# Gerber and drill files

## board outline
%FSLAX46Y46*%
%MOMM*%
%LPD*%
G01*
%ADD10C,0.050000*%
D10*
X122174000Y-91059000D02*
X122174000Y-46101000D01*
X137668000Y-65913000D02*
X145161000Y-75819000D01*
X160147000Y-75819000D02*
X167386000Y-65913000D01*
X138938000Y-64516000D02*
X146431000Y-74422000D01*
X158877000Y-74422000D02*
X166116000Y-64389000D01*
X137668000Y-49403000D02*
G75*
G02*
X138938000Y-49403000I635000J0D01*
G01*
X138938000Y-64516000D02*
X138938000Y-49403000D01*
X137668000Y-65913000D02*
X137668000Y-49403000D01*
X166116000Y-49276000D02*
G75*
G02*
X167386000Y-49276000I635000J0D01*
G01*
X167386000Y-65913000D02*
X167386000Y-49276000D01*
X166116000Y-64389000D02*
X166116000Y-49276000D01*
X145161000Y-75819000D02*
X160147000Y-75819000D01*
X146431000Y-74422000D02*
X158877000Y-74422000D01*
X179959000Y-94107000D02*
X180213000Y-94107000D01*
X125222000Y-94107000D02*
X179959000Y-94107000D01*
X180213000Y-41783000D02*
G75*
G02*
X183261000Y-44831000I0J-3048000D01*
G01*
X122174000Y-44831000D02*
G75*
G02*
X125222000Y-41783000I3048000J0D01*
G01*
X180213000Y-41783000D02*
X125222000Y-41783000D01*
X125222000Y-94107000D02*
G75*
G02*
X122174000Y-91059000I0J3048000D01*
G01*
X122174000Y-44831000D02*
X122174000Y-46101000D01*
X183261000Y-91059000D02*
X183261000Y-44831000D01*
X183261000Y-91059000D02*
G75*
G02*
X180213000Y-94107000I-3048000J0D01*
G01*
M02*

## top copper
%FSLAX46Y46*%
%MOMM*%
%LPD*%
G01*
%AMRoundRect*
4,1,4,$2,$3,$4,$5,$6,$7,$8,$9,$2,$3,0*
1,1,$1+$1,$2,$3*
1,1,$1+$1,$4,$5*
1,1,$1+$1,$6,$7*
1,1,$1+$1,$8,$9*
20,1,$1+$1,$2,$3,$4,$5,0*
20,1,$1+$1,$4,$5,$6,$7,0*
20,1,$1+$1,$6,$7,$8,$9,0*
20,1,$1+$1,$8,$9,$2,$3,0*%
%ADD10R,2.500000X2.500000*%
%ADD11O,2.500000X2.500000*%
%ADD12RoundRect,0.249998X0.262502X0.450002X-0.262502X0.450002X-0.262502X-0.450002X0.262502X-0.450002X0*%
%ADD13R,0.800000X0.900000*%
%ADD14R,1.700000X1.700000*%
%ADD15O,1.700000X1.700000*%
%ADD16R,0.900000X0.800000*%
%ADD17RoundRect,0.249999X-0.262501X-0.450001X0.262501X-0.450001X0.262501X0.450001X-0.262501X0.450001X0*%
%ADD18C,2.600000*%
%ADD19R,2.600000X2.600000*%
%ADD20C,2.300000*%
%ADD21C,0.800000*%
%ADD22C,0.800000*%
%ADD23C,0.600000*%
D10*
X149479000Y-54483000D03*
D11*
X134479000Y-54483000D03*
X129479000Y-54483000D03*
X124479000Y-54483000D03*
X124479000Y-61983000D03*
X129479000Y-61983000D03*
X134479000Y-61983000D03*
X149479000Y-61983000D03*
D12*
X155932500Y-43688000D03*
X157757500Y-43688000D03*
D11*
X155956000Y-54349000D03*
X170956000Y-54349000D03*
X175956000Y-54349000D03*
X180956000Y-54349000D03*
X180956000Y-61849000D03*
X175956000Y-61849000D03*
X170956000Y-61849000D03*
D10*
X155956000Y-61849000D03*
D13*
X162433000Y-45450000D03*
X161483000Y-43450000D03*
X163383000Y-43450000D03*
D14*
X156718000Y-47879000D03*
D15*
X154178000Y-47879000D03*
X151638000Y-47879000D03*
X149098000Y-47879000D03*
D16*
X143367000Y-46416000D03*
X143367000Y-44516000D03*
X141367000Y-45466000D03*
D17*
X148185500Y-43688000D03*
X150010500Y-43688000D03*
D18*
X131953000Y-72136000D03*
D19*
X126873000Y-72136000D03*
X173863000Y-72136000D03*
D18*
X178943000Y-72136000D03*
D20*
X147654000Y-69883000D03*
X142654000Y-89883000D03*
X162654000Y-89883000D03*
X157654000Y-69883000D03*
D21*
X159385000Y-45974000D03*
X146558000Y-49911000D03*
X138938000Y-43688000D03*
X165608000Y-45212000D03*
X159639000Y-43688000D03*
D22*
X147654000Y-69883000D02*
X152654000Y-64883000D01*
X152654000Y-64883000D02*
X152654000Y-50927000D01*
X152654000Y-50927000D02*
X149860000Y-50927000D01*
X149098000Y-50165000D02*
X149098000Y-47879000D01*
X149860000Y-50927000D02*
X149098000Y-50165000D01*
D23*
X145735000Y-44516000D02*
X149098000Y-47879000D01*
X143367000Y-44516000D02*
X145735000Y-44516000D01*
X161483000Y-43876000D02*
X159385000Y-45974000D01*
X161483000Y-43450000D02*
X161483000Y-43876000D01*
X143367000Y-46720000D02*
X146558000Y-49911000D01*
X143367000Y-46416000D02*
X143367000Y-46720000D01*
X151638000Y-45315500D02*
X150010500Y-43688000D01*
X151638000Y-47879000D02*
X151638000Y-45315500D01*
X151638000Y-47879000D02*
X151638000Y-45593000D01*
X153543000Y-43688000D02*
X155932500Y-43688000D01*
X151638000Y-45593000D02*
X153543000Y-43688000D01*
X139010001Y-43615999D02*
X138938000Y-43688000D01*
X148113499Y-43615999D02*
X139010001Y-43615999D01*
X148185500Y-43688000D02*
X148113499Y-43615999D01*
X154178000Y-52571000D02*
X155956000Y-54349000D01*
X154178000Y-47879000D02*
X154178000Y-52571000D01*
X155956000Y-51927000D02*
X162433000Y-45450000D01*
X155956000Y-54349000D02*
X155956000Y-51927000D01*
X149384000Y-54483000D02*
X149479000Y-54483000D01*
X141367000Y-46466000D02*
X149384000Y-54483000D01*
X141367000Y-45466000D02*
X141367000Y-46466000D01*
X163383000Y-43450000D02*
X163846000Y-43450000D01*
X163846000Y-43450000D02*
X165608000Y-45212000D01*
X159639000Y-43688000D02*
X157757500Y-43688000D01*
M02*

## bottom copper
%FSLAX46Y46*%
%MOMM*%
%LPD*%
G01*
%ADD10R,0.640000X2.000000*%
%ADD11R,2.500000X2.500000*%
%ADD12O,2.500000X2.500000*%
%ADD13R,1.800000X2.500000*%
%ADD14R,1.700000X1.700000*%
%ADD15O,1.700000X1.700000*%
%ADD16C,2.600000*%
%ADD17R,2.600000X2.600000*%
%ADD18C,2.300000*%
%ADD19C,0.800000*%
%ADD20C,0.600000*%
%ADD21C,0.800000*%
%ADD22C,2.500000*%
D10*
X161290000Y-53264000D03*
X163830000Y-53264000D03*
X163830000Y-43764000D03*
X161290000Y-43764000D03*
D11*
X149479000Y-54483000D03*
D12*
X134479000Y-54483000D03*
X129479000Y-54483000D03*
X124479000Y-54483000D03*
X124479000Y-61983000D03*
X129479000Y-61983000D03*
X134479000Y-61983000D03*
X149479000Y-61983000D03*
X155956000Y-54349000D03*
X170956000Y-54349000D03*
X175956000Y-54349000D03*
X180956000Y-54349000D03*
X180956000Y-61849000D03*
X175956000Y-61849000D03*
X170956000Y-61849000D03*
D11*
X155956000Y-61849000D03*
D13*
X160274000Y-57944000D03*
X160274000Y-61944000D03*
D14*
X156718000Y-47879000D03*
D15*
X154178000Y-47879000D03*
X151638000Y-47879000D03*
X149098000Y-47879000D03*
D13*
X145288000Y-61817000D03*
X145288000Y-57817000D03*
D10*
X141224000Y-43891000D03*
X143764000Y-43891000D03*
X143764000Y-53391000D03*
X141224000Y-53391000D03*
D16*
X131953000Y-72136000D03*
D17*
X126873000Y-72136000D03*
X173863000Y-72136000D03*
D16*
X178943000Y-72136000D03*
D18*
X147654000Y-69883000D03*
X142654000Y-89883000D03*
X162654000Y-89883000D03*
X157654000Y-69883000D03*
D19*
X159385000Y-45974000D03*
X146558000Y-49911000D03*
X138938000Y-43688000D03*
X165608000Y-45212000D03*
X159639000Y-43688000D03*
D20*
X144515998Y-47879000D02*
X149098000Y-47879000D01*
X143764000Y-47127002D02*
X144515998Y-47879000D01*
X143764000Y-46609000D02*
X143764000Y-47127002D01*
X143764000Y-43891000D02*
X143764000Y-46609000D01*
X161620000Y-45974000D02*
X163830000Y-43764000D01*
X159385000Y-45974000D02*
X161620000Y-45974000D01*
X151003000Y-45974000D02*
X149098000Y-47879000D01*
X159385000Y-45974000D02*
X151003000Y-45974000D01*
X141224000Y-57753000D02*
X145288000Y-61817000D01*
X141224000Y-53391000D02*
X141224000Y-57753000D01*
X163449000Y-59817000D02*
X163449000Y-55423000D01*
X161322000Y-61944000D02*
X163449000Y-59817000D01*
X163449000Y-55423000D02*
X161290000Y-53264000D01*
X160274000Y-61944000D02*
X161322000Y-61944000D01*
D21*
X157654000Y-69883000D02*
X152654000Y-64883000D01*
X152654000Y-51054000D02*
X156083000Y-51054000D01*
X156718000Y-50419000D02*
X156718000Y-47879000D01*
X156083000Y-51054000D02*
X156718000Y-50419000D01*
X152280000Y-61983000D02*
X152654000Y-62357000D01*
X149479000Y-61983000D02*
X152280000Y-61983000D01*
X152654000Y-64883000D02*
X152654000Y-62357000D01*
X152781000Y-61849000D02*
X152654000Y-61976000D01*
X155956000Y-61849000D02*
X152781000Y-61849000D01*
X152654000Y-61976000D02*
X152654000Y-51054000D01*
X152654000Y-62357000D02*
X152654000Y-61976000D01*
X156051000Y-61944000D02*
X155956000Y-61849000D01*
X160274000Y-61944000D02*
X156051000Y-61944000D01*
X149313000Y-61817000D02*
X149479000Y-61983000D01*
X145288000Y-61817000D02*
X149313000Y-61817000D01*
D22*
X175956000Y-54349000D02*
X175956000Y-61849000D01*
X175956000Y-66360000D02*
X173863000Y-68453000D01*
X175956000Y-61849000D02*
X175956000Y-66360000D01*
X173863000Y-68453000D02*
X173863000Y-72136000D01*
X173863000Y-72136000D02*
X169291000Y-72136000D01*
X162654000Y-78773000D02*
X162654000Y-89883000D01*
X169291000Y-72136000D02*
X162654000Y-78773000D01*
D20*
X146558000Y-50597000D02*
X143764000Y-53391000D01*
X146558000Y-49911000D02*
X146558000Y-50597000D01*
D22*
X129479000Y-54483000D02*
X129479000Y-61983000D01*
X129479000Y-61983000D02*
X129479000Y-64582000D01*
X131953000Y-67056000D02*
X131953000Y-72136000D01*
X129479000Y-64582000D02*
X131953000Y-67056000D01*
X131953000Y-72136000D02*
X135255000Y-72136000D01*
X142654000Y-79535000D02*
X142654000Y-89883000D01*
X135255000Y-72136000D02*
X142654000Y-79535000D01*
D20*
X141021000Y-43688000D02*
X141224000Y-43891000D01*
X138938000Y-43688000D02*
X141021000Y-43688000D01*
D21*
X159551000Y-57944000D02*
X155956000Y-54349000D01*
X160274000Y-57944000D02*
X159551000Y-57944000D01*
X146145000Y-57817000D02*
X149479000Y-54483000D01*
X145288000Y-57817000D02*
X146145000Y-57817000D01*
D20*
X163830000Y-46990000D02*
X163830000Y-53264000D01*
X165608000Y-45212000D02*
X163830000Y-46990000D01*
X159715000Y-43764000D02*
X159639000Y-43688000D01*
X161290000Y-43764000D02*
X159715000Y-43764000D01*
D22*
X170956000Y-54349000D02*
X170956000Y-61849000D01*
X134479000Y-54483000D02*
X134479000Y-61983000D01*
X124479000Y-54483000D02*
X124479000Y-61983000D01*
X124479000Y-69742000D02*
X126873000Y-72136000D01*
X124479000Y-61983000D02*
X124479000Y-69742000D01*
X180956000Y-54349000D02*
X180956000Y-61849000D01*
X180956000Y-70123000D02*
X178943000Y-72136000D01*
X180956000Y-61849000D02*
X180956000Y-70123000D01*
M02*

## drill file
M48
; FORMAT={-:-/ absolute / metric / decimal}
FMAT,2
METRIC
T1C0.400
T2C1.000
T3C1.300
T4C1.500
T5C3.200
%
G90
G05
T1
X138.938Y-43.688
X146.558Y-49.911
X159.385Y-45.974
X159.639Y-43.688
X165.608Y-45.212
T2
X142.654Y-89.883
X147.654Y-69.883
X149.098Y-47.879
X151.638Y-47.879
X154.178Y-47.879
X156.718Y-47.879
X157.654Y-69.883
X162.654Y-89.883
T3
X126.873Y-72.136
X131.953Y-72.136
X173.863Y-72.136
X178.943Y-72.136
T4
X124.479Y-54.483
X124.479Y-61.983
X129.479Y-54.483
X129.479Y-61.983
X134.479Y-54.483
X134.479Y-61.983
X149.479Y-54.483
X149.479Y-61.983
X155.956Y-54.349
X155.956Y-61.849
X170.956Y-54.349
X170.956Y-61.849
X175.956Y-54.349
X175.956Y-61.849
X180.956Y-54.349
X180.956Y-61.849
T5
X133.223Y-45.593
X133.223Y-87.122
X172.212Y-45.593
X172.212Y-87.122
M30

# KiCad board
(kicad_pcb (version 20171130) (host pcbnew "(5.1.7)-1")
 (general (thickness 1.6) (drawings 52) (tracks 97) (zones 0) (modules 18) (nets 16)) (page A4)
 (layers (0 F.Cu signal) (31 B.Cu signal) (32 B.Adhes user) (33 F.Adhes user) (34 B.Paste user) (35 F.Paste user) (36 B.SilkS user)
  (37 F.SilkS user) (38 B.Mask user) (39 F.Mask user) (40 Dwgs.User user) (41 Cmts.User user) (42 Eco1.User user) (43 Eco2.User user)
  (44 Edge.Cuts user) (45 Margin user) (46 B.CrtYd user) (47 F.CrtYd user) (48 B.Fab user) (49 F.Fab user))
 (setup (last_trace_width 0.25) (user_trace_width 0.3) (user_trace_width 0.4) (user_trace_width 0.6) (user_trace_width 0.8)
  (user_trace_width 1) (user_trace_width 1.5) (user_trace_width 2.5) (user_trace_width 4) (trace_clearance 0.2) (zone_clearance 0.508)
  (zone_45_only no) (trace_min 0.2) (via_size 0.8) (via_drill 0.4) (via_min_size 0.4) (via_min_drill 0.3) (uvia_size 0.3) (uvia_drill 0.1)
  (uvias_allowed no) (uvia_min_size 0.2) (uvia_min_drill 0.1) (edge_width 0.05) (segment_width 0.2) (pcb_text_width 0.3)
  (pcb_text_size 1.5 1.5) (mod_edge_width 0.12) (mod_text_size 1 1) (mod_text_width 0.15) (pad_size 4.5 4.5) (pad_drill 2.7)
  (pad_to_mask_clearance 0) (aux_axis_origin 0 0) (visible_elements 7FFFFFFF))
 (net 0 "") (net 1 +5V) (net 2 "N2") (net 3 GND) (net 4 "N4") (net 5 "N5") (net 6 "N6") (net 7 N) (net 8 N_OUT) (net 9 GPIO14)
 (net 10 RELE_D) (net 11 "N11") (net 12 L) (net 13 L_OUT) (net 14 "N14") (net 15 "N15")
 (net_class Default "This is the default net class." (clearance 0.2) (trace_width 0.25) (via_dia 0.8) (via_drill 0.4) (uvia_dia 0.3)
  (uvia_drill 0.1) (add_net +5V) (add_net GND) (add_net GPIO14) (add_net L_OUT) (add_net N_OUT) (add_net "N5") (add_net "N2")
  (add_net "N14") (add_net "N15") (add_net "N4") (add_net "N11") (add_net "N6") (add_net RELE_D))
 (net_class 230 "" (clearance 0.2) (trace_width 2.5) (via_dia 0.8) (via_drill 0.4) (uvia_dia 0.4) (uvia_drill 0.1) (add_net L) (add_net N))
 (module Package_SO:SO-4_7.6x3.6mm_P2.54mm (layer B.Cu) (at 162.56 48.514 270)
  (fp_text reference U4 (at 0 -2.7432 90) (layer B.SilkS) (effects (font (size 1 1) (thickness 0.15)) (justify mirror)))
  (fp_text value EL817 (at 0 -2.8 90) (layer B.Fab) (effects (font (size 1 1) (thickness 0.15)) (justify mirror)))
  (pad 4 smd rect (at 4.75 1.27 270) (size 2 0.64) (layers B.Cu B.Paste B.Mask) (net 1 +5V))
  (pad 3 smd rect (at 4.75 -1.27 270) (size 2 0.64) (layers B.Cu B.Paste B.Mask) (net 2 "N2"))
  (pad 2 smd rect (at -4.75 -1.27 270) (size 2 0.64) (layers B.Cu B.Paste B.Mask) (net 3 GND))
  (pad 1 smd rect (at -4.75 1.27 270) (size 2 0.64) (layers B.Cu B.Paste B.Mask) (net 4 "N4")))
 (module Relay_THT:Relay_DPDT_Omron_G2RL (layer F.Cu) (at 149.479 54.483 180)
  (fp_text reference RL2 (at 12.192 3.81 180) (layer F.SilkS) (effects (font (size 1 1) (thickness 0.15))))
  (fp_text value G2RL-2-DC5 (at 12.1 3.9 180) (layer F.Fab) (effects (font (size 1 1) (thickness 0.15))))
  (pad 1 thru_hole rect (at 0 0 270) (size 2.5 2.5) (drill 1.5) (layers *.Cu *.Mask) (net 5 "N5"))
  (pad 2 thru_hole oval (at 15 0 270) (size 2.5 2.5) (drill 1.5) (layers *.Cu *.Mask) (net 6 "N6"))
  (pad 3 thru_hole oval (at 20 0 270) (size 2.5 2.5) (drill 1.5) (layers *.Cu *.Mask) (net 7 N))
  (pad 4 thru_hole oval (at 25 0 270) (size 2.5 2.5) (drill 1.5) (layers *.Cu *.Mask) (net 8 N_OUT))
  (pad 5 thru_hole oval (at 25 -7.5 270) (size 2.5 2.5) (drill 1.5) (layers *.Cu *.Mask) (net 8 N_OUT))
  (pad 6 thru_hole oval (at 20 -7.5 270) (size 2.5 2.5) (drill 1.5) (layers *.Cu *.Mask) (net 7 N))
  (pad 7 thru_hole oval (at 15 -7.5 270) (size 2.5 2.5) (drill 1.5) (layers *.Cu *.Mask) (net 6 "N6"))
  (pad 8 thru_hole oval (at 0 -7.5 270) (size 2.5 2.5) (drill 1.5) (layers *.Cu *.Mask) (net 1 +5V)))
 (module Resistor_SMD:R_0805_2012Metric (layer F.Cu) (at 156.845 43.688 180)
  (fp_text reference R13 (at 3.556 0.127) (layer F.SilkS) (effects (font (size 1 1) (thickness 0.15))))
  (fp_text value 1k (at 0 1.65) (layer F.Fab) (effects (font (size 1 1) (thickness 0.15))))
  (pad 2 smd roundrect (at 0.9125 0 180) (size 1.025 1.4) (layers F.Cu F.Paste F.Mask) (roundrect_rratio 0.2439004878048781) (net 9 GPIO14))
  (pad 1 smd roundrect (at -0.9125 0 180) (size 1.025 1.4) (layers F.Cu F.Paste F.Mask) (roundrect_rratio 0.2439004878048781) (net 4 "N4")))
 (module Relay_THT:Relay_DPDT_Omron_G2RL (layer F.Cu) (at 155.956 61.849)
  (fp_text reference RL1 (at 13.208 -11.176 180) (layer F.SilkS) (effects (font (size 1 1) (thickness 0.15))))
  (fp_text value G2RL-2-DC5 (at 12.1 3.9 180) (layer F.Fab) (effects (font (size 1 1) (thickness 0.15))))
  (pad 8 thru_hole oval (at 0 -7.5 90) (size 2.5 2.5) (drill 1.5) (layers *.Cu *.Mask) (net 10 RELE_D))
  (pad 7 thru_hole oval (at 15 -7.5 90) (size 2.5 2.5) (drill 1.5) (layers *.Cu *.Mask) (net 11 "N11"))
  (pad 6 thru_hole oval (at 20 -7.5 90) (size 2.5 2.5) (drill 1.5) (layers *.Cu *.Mask) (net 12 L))
  (pad 5 thru_hole oval (at 25 -7.5 90) (size 2.5 2.5) (drill 1.5) (layers *.Cu *.Mask) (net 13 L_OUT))
  (pad 4 thru_hole oval (at 25 0 90) (size 2.5 2.5) (drill 1.5) (layers *.Cu *.Mask) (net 13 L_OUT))
  (pad 3 thru_hole oval (at 20 0 90) (size 2.5 2.5) (drill 1.5) (layers *.Cu *.Mask) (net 12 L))
  (pad 2 thru_hole oval (at 15 0 90) (size 2.5 2.5) (drill 1.5) (layers *.Cu *.Mask) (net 11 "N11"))
  (pad 1 thru_hole rect (at 0 0 90) (size 2.5 2.5) (drill 1.5) (layers *.Cu *.Mask) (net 1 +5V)))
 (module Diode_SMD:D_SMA (layer B.Cu) (at 160.274 59.944 90)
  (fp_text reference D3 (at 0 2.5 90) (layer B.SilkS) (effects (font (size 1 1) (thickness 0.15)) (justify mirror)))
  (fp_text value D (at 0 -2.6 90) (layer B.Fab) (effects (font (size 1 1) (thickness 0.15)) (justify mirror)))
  (pad 2 smd rect (at 2 0 90) (size 2.5 1.8) (layers B.Cu B.Paste B.Mask) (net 10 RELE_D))
  (pad 1 smd rect (at -2 0 90) (size 2.5 1.8) (layers B.Cu B.Paste B.Mask) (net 1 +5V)))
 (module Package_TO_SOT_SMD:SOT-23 (layer F.Cu) (at 162.433 44.45 270)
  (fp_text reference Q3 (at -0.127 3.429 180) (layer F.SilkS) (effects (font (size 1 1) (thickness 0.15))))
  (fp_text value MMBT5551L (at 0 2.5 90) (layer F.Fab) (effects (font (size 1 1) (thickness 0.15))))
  (pad 3 smd rect (at 1 0 270) (size 0.9 0.8) (layers F.Cu F.Paste F.Mask) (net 10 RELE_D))
  (pad 2 smd rect (at -1 0.95 270) (size 0.9 0.8) (layers F.Cu F.Paste F.Mask) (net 3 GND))
  (pad 1 smd rect (at -1 -0.95 270) (size 0.9 0.8) (layers F.Cu F.Paste F.Mask) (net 2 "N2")))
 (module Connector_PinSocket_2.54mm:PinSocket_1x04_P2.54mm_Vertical (layer F.Cu) (at 156.718 47.879 270)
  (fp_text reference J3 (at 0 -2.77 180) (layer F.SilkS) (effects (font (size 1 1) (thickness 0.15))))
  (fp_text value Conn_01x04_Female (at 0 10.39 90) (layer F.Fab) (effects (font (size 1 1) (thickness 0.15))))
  (pad 1 thru_hole rect (at 0 0 270) (size 1.7 1.7) (drill 1) (layers *.Cu *.Mask) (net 1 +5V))
  (pad 2 thru_hole oval (at 0 2.54 270) (size 1.7 1.7) (drill 1) (layers *.Cu *.Mask) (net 10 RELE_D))
  (pad 3 thru_hole oval (at 0 5.08 270) (size 1.7 1.7) (drill 1) (layers *.Cu *.Mask) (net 9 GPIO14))
  (pad 4 thru_hole oval (at 0 7.62 270) (size 1.7 1.7) (drill 1) (layers *.Cu *.Mask) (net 3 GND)))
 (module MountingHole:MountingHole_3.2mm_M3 (layer F.Cu) (at 133.223 45.593)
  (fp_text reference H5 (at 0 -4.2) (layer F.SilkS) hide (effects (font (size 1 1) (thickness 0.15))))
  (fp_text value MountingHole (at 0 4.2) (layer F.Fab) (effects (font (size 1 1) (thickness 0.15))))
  (pad 1 np_thru_hole circle (at 0 0) (size 3.2 3.2) (drill 3.2) (layers *.Cu *.Mask)))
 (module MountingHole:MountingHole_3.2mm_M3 (layer F.Cu) (at 172.212 45.593)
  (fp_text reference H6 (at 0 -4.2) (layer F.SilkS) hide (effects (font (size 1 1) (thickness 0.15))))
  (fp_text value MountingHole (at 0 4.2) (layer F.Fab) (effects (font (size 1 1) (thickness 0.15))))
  (pad 1 np_thru_hole circle (at 0 0) (size 3.2 3.2) (drill 3.2) (layers *.Cu *.Mask)))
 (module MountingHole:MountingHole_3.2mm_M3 (layer F.Cu) (at 133.223 87.122)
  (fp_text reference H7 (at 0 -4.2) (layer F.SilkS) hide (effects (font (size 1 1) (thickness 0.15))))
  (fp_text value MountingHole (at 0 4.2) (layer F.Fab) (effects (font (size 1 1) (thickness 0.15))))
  (pad 1 np_thru_hole circle (at 0 0) (size 3.2 3.2) (drill 3.2) (layers *.Cu *.Mask)))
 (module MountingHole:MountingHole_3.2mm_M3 (layer F.Cu) (at 172.212 87.122)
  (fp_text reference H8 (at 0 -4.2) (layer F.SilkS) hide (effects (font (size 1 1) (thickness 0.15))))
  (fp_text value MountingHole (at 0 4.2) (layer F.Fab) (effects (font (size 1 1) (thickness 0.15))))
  (pad 1 np_thru_hole circle (at 0 0) (size 3.2 3.2) (drill 3.2) (layers *.Cu *.Mask)))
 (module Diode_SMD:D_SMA (layer B.Cu) (at 145.288 59.817 90)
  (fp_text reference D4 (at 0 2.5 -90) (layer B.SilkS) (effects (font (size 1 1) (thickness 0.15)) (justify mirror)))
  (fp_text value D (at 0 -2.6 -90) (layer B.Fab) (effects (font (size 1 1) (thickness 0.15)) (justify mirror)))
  (pad 1 smd rect (at -2 0 90) (size 2.5 1.8) (layers B.Cu B.Paste B.Mask) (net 1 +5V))
  (pad 2 smd rect (at 2 0 90) (size 2.5 1.8) (layers B.Cu B.Paste B.Mask) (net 5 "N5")))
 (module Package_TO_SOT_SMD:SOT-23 (layer F.Cu) (at 142.367 45.466 180)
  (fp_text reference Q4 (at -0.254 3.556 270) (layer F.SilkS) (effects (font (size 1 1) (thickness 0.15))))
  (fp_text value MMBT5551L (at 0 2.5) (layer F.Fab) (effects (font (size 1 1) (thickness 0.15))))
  (pad 1 smd rect (at -1 -0.95 180) (size 0.9 0.8) (layers F.Cu F.Paste F.Mask) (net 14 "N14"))
  (pad 2 smd rect (at -1 0.95 180) (size 0.9 0.8) (layers F.Cu F.Paste F.Mask) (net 3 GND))
  (pad 3 smd rect (at 1 0 180) (size 0.9 0.8) (layers F.Cu F.Paste F.Mask) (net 5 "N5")))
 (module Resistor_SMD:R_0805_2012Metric (layer F.Cu) (at 149.098 43.688)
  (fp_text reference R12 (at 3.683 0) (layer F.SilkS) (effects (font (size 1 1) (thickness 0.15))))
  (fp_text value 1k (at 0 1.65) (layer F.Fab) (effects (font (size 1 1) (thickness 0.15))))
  (pad 1 smd roundrect (at -0.9125 0) (size 1.025 1.4) (layers F.Cu F.Paste F.Mask) (roundrect_rratio 0.2439014634146341) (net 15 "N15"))
  (pad 2 smd roundrect (at 0.9125 0) (size 1.025 1.4) (layers F.Cu F.Paste F.Mask) (roundrect_rratio 0.2439014634146341) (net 9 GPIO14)))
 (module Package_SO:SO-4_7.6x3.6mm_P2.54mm (layer B.Cu) (at 142.494 48.641 270)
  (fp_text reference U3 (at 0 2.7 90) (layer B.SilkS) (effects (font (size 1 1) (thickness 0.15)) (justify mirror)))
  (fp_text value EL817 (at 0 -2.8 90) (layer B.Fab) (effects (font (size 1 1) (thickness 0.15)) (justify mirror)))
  (pad 1 smd rect (at -4.75 1.27 270) (size 2 0.64) (layers B.Cu B.Paste B.Mask) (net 15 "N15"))
  (pad 2 smd rect (at -4.75 -1.27 270) (size 2 0.64) (layers B.Cu B.Paste B.Mask) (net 3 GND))
  (pad 3 smd rect (at 4.75 -1.27 270) (size 2 0.64) (layers B.Cu B.Paste B.Mask) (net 14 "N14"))
  (pad 4 smd rect (at 4.75 1.27 270) (size 2 0.64) (layers B.Cu B.Paste B.Mask) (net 1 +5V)))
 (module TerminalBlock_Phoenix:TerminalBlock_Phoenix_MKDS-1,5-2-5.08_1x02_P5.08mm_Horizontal (layer F.Cu) (at 126.873 72.136)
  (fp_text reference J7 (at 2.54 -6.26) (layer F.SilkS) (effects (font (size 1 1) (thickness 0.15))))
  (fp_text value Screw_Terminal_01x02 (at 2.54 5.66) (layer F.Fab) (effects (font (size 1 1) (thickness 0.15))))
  (pad 2 thru_hole circle (at 5.08 0) (size 2.6 2.6) (drill 1.3) (layers *.Cu *.Mask) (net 7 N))
  (pad 1 thru_hole rect (at 0 0) (size 2.6 2.6) (drill 1.3) (layers *.Cu *.Mask) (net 8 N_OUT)))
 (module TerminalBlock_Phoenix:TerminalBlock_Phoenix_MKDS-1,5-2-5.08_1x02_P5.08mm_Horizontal (layer F.Cu) (at 173.863 72.136)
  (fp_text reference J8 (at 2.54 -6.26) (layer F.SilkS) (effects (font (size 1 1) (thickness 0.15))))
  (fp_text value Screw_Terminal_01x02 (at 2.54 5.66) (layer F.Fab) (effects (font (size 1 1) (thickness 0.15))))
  (pad 1 thru_hole rect (at 0 0) (size 2.6 2.6) (drill 1.3) (layers *.Cu *.Mask) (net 12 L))
  (pad 2 thru_hole circle (at 5.08 0) (size 2.6 2.6) (drill 1.3) (layers *.Cu *.Mask) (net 13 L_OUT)))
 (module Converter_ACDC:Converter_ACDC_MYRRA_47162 (layer F.Cu) (at 152.654 79.883 180)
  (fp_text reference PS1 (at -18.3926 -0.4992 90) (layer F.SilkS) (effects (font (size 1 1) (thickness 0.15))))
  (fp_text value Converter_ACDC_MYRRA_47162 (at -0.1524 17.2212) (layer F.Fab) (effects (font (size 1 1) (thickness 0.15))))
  (pad 9 thru_hole circle (at 5 10 180) (size 2.3 2.3) (drill 1) (layers *.Cu *.Mask) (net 3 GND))
  (pad 1 thru_hole circle (at 10 -10 180) (size 2.3 2.3) (drill 1) (layers *.Cu *.Mask) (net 7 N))
  (pad 5 thru_hole circle (at -10 -10 180) (size 2.3 2.3) (drill 1) (layers *.Cu *.Mask) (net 12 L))
  (pad 7 thru_hole circle (at -5 10 180) (size 2.3 2.3) (drill 1) (layers *.Cu *.Mask) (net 1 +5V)))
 (gr_line (start 122.174 91.059) (end 122.174 46.101) (layer Edge.Cuts) (width 0.05))
 (gr_line (start 137.668 65.913) (end 145.161 75.819) (layer Edge.Cuts) (width 0.05))
 (gr_line (start 160.147 75.819) (end 167.386 65.913) (layer Edge.Cuts) (width 0.05))
 (gr_line (start 138.938 64.516) (end 146.431 74.422) (layer Edge.Cuts) (width 0.05))
 (gr_line (start 158.877 74.422) (end 166.116 64.389) (layer Edge.Cuts) (width 0.05))
 (gr_arc (start 138.303 49.403) (end 138.938 49.403) (angle -180) (layer Edge.Cuts) (width 0.05))
 (gr_line (start 138.938 64.516) (end 138.938 49.403) (layer Edge.Cuts) (width 0.05))
 (gr_line (start 137.668 65.913) (end 137.668 49.403) (layer Edge.Cuts) (width 0.05))
 (gr_arc (start 166.751 49.276) (end 167.386 49.276) (angle -180) (layer Edge.Cuts) (width 0.05))
 (gr_line (start 167.386 65.913) (end 167.386 49.276) (layer Edge.Cuts) (width 0.05))
 (gr_line (start 166.116 64.389) (end 166.116 49.276) (layer Edge.Cuts) (width 0.05))
 (gr_line (start 145.161 75.819) (end 160.147 75.819) (layer Edge.Cuts) (width 0.05))
 (gr_line (start 146.431 74.422) (end 158.877 74.422) (layer Edge.Cuts) (width 0.05))
 (gr_line (start 179.959 94.107) (end 180.213 94.107) (layer Edge.Cuts) (width 0.05))
 (gr_line (start 125.222 94.107) (end 179.959 94.107) (layer Edge.Cuts) (width 0.05))
 (gr_arc (start 180.213 44.831) (end 183.261 44.831) (angle -90) (layer Edge.Cuts) (width 0.05))
 (gr_arc (start 125.222 44.831) (end 125.222 41.783) (angle -90) (layer Edge.Cuts) (width 0.05))
 (gr_line (start 180.213 41.783) (end 125.222 41.783) (layer Edge.Cuts) (width 0.05))
 (gr_arc (start 125.222 91.059) (end 122.174 91.059) (angle -90) (layer Edge.Cuts) (width 0.05))
 (gr_line (start 122.174 44.831) (end 122.174 46.101) (layer Edge.Cuts) (width 0.05))
 (gr_line (start 183.261 91.059) (end 183.261 44.831) (layer Edge.Cuts) (width 0.05))
 (gr_arc (start 180.213 91.059) (end 180.213 94.107) (angle -90) (layer Edge.Cuts) (width 0.05))
 (segment (start 144.515998 47.879) (end 149.098 47.879) (width 0.6) (layer B.Cu) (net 3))
 (segment (start 143.764 47.127002) (end 144.515998 47.879) (width 0.6) (layer B.Cu) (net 3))
 (segment (start 147.654 69.883) (end 152.654 64.883) (width 0.8) (layer F.Cu) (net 3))
 (segment (start 152.654 64.883) (end 152.654 50.927) (width 0.8) (layer F.Cu) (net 3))
 (segment (start 152.654 50.927) (end 149.86 50.927) (width 0.8) (layer F.Cu) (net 3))
 (segment (start 149.098 50.165) (end 149.098 47.879) (width 0.8) (layer F.Cu) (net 3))
 (segment (start 149.86 50.927) (end 149.098 50.165) (width 0.8) (layer F.Cu) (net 3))
 (segment (start 143.764 46.609) (end 143.764 47.127002) (width 0.6) (layer B.Cu) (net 3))
 (segment (start 143.764 43.891) (end 143.764 46.609) (width 0.6) (layer B.Cu) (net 3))
 (segment (start 145.735 44.516) (end 149.098 47.879) (width 0.6) (layer F.Cu) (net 3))
 (segment (start 143.367 44.516) (end 145.735 44.516) (width 0.6) (layer F.Cu) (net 3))
 (via (at 159.385 45.974) (size 0.8) (drill 0.4) (layers F.Cu B.Cu) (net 3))
 (segment (start 161.483 43.876) (end 159.385 45.974) (width 0.6) (layer F.Cu) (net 3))
 (segment (start 161.483 43.45) (end 161.483 43.876) (width 0.6) (layer F.Cu) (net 3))
 (segment (start 161.62 45.974) (end 163.83 43.764) (width 0.6) (layer B.Cu) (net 3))
 (segment (start 159.385 45.974) (end 161.62 45.974) (width 0.6) (layer B.Cu) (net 3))
 (segment (start 151.003 45.974) (end 149.098 47.879) (width 0.6) (layer B.Cu) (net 3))
 (segment (start 159.385 45.974) (end 151.003 45.974) (width 0.6) (layer B.Cu) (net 3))
 (segment (start 141.224 57.753) (end 145.288 61.817) (width 0.6) (layer B.Cu) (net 1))
 (segment (start 141.224 53.391) (end 141.224 57.753) (width 0.6) (layer B.Cu) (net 1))
 (segment (start 163.449 59.817) (end 163.449 55.423) (width 0.6) (layer B.Cu) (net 1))
 (segment (start 161.322 61.944) (end 163.449 59.817) (width 0.6) (layer B.Cu) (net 1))
 (segment (start 163.449 55.423) (end 161.29 53.264) (width 0.6) (layer B.Cu) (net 1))
 (segment (start 160.274 61.944) (end 161.322 61.944) (width 0.6) (layer B.Cu) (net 1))
 (segment (start 157.654 69.883) (end 152.654 64.883) (width 0.8) (layer B.Cu) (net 1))
 (segment (start 152.654 51.054) (end 156.083 51.054) (width 0.8) (layer B.Cu) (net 1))
 (segment (start 156.718 50.419) (end 156.718 47.879) (width 0.8) (layer B.Cu) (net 1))
 (segment (start 156.083 51.054) (end 156.718 50.419) (width 0.8) (layer B.Cu) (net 1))
 (segment (start 152.28 61.983) (end 152.654 62.357) (width 0.8) (layer B.Cu) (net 1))
 (segment (start 149.479 61.983) (end 152.28 61.983) (width 0.8) (layer B.Cu) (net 1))
 (segment (start 152.654 64.883) (end 152.654 62.357) (width 0.8) (layer B.Cu) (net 1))
 (segment (start 152.781 61.849) (end 152.654 61.976) (width 0.8) (layer B.Cu) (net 1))
 (segment (start 155.956 61.849) (end 152.781 61.849) (width 0.8) (layer B.Cu) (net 1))
 (segment (start 152.654 61.976) (end 152.654 51.054) (width 0.8) (layer B.Cu) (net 1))
 (segment (start 152.654 62.357) (end 152.654 61.976) (width 0.8) (layer B.Cu) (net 1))
 (segment (start 156.051 61.944) (end 155.956 61.849) (width 0.8) (layer B.Cu) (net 1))
 (segment (start 160.274 61.944) (end 156.051 61.944) (width 0.8) (layer B.Cu) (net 1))
 (segment (start 149.313 61.817) (end 149.479 61.983) (width 0.8) (layer B.Cu) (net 1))
 (segment (start 145.288 61.817) (end 149.313 61.817) (width 0.8) (layer B.Cu) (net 1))
 (segment (start 175.956 54.349) (end 175.956 61.849) (width 2.5) (layer B.Cu) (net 12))
 (segment (start 175.956 66.36) (end 173.863 68.453) (width 2.5) (layer B.Cu) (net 12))
 (segment (start 175.956 61.849) (end 175.956 66.36) (width 2.5) (layer B.Cu) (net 12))
 (segment (start 173.863 68.453) (end 173.863 72.136) (width 2.5) (layer B.Cu) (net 12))
 (segment (start 173.863 72.136) (end 169.291 72.136) (width 2.5) (layer B.Cu) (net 12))
 (segment (start 162.654 78.773) (end 162.654 89.883) (width 2.5) (layer B.Cu) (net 12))
 (segment (start 169.291 72.136) (end 162.654 78.773) (width 2.5) (layer B.Cu) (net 12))
 (via (at 146.558 49.911) (size 0.8) (drill 0.4) (layers F.Cu B.Cu) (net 14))
 (segment (start 143.367 46.72) (end 146.558 49.911) (width 0.6) (layer F.Cu) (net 14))
 (segment (start 143.367 46.416) (end 143.367 46.72) (width 0.6) (layer F.Cu) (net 14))
 (segment (start 146.558 50.597) (end 143.764 53.391) (width 0.6) (layer B.Cu) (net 14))
 (segment (start 146.558 49.911) (end 146.558 50.597) (width 0.6) (layer B.Cu) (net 14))
 (segment (start 129.479 54.483) (end 129.479 61.983) (width 2.5) (layer B.Cu) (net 7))
 (segment (start 129.479 61.983) (end 129.479 64.582) (width 2.5) (layer B.Cu) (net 7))
 (segment (start 131.953 67.056) (end 131.953 72.136) (width 2.5) (layer B.Cu) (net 7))
 (segment (start 129.479 64.582) (end 131.953 67.056) (width 2.5) (layer B.Cu) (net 7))
 (segment (start 131.953 72.136) (end 135.255 72.136) (width 2.5) (layer B.Cu) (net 7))
 (segment (start 142.654 79.535) (end 142.654 89.883) (width 2.5) (layer B.Cu) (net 7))
 (segment (start 135.255 72.136) (end 142.654 79.535) (width 2.5) (layer B.Cu) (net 7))
 (segment (start 151.638 45.3155) (end 150.0105 43.688) (width 0.6) (layer F.Cu) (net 9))
 (segment (start 151.638 47.879) (end 151.638 45.3155) (width 0.6) (layer F.Cu) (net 9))
 (segment (start 151.638 47.879) (end 151.638 45.593) (width 0.6) (layer F.Cu) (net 9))
 (segment (start 153.543 43.688) (end 155.9325 43.688) (width 0.6) (layer F.Cu) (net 9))
 (segment (start 151.638 45.593) (end 153.543 43.688) (width 0.6) (layer F.Cu) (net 9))
 (via (at 138.938 43.688) (size 0.8) (drill 0.4) (layers F.Cu B.Cu) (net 15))
 (segment (start 139.010001 43.615999) (end 138.938 43.688) (width 0.6) (layer F.Cu) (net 15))
 (segment (start 148.113499 43.615999) (end 139.010001 43.615999) (width 0.6) (layer F.Cu) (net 15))
 (segment (start 148.1855 43.688) (end 148.113499 43.615999) (width 0.6) (layer F.Cu) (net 15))
 (segment (start 141.021 43.688) (end 141.224 43.891) (width 0.6) (layer B.Cu) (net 15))
 (segment (start 138.938 43.688) (end 141.021 43.688) (width 0.6) (layer B.Cu) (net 15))
 (segment (start 159.551 57.944) (end 155.956 54.349) (width 0.8) (layer B.Cu) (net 10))
 (segment (start 160.274 57.944) (end 159.551 57.944) (width 0.8) (layer B.Cu) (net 10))
 (segment (start 154.178 52.571) (end 155.956 54.349) (width 0.6) (layer F.Cu) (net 10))
 (segment (start 154.178 47.879) (end 154.178 52.571) (width 0.6) (layer F.Cu) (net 10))
 (segment (start 155.956 51.927) (end 162.433 45.45) (width 0.6) (layer F.Cu) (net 10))
 (segment (start 155.956 54.349) (end 155.956 51.927) (width 0.6) (layer F.Cu) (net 10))
 (segment (start 146.145 57.817) (end 149.479 54.483) (width 0.8) (layer B.Cu) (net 5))
 (segment (start 145.288 57.817) (end 146.145 57.817) (width 0.8) (layer B.Cu) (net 5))
 (segment (start 149.384 54.483) (end 149.479 54.483) (width 0.6) (layer F.Cu) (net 5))
 (segment (start 141.367 46.466) (end 149.384 54.483) (width 0.6) (layer F.Cu) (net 5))
 (segment (start 141.367 45.466) (end 141.367 46.466) (width 0.6) (layer F.Cu) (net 5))
 (segment (start 163.383 43.45) (end 163.846 43.45) (width 0.6) (layer F.Cu) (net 2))
 (via (at 165.608 45.212) (size 0.8) (drill 0.4) (layers F.Cu B.Cu) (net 2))
 (segment (start 163.846 43.45) (end 165.608 45.212) (width 0.6) (layer F.Cu) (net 2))
 (segment (start 163.83 46.99) (end 163.83 53.264) (width 0.6) (layer B.Cu) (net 2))
 (segment (start 165.608 45.212) (end 163.83 46.99) (width 0.6) (layer B.Cu) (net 2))
 (via (at 159.639 43.688) (size 0.8) (drill 0.4) (layers F.Cu B.Cu) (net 4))
 (segment (start 159.715 43.764) (end 159.639 43.688) (width 0.6) (layer B.Cu) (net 4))
 (segment (start 161.29 43.764) (end 159.715 43.764) (width 0.6) (layer B.Cu) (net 4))
 (segment (start 159.639 43.688) (end 157.7575 43.688) (width 0.6) (layer F.Cu) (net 4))
 (segment (start 170.956 54.349) (end 170.956 61.849) (width 2.5) (layer B.Cu) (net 11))
 (segment (start 134.479 54.483) (end 134.479 61.983) (width 2.5) (layer B.Cu) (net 6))
 (segment (start 124.479 54.483) (end 124.479 61.983) (width 2.5) (layer B.Cu) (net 8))
 (segment (start 124.479 69.742) (end 126.873 72.136) (width 2.5) (layer B.Cu) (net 8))
 (segment (start 124.479 61.983) (end 124.479 69.742) (width 2.5) (layer B.Cu) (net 8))
 (segment (start 180.956 54.349) (end 180.956 61.849) (width 2.5) (layer B.Cu) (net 13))
 (segment (start 180.956 70.123) (end 178.943 72.136) (width 2.5) (layer B.Cu) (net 13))
 (segment (start 180.956 61.849) (end 180.956 70.123) (width 2.5) (layer B.Cu) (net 13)))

